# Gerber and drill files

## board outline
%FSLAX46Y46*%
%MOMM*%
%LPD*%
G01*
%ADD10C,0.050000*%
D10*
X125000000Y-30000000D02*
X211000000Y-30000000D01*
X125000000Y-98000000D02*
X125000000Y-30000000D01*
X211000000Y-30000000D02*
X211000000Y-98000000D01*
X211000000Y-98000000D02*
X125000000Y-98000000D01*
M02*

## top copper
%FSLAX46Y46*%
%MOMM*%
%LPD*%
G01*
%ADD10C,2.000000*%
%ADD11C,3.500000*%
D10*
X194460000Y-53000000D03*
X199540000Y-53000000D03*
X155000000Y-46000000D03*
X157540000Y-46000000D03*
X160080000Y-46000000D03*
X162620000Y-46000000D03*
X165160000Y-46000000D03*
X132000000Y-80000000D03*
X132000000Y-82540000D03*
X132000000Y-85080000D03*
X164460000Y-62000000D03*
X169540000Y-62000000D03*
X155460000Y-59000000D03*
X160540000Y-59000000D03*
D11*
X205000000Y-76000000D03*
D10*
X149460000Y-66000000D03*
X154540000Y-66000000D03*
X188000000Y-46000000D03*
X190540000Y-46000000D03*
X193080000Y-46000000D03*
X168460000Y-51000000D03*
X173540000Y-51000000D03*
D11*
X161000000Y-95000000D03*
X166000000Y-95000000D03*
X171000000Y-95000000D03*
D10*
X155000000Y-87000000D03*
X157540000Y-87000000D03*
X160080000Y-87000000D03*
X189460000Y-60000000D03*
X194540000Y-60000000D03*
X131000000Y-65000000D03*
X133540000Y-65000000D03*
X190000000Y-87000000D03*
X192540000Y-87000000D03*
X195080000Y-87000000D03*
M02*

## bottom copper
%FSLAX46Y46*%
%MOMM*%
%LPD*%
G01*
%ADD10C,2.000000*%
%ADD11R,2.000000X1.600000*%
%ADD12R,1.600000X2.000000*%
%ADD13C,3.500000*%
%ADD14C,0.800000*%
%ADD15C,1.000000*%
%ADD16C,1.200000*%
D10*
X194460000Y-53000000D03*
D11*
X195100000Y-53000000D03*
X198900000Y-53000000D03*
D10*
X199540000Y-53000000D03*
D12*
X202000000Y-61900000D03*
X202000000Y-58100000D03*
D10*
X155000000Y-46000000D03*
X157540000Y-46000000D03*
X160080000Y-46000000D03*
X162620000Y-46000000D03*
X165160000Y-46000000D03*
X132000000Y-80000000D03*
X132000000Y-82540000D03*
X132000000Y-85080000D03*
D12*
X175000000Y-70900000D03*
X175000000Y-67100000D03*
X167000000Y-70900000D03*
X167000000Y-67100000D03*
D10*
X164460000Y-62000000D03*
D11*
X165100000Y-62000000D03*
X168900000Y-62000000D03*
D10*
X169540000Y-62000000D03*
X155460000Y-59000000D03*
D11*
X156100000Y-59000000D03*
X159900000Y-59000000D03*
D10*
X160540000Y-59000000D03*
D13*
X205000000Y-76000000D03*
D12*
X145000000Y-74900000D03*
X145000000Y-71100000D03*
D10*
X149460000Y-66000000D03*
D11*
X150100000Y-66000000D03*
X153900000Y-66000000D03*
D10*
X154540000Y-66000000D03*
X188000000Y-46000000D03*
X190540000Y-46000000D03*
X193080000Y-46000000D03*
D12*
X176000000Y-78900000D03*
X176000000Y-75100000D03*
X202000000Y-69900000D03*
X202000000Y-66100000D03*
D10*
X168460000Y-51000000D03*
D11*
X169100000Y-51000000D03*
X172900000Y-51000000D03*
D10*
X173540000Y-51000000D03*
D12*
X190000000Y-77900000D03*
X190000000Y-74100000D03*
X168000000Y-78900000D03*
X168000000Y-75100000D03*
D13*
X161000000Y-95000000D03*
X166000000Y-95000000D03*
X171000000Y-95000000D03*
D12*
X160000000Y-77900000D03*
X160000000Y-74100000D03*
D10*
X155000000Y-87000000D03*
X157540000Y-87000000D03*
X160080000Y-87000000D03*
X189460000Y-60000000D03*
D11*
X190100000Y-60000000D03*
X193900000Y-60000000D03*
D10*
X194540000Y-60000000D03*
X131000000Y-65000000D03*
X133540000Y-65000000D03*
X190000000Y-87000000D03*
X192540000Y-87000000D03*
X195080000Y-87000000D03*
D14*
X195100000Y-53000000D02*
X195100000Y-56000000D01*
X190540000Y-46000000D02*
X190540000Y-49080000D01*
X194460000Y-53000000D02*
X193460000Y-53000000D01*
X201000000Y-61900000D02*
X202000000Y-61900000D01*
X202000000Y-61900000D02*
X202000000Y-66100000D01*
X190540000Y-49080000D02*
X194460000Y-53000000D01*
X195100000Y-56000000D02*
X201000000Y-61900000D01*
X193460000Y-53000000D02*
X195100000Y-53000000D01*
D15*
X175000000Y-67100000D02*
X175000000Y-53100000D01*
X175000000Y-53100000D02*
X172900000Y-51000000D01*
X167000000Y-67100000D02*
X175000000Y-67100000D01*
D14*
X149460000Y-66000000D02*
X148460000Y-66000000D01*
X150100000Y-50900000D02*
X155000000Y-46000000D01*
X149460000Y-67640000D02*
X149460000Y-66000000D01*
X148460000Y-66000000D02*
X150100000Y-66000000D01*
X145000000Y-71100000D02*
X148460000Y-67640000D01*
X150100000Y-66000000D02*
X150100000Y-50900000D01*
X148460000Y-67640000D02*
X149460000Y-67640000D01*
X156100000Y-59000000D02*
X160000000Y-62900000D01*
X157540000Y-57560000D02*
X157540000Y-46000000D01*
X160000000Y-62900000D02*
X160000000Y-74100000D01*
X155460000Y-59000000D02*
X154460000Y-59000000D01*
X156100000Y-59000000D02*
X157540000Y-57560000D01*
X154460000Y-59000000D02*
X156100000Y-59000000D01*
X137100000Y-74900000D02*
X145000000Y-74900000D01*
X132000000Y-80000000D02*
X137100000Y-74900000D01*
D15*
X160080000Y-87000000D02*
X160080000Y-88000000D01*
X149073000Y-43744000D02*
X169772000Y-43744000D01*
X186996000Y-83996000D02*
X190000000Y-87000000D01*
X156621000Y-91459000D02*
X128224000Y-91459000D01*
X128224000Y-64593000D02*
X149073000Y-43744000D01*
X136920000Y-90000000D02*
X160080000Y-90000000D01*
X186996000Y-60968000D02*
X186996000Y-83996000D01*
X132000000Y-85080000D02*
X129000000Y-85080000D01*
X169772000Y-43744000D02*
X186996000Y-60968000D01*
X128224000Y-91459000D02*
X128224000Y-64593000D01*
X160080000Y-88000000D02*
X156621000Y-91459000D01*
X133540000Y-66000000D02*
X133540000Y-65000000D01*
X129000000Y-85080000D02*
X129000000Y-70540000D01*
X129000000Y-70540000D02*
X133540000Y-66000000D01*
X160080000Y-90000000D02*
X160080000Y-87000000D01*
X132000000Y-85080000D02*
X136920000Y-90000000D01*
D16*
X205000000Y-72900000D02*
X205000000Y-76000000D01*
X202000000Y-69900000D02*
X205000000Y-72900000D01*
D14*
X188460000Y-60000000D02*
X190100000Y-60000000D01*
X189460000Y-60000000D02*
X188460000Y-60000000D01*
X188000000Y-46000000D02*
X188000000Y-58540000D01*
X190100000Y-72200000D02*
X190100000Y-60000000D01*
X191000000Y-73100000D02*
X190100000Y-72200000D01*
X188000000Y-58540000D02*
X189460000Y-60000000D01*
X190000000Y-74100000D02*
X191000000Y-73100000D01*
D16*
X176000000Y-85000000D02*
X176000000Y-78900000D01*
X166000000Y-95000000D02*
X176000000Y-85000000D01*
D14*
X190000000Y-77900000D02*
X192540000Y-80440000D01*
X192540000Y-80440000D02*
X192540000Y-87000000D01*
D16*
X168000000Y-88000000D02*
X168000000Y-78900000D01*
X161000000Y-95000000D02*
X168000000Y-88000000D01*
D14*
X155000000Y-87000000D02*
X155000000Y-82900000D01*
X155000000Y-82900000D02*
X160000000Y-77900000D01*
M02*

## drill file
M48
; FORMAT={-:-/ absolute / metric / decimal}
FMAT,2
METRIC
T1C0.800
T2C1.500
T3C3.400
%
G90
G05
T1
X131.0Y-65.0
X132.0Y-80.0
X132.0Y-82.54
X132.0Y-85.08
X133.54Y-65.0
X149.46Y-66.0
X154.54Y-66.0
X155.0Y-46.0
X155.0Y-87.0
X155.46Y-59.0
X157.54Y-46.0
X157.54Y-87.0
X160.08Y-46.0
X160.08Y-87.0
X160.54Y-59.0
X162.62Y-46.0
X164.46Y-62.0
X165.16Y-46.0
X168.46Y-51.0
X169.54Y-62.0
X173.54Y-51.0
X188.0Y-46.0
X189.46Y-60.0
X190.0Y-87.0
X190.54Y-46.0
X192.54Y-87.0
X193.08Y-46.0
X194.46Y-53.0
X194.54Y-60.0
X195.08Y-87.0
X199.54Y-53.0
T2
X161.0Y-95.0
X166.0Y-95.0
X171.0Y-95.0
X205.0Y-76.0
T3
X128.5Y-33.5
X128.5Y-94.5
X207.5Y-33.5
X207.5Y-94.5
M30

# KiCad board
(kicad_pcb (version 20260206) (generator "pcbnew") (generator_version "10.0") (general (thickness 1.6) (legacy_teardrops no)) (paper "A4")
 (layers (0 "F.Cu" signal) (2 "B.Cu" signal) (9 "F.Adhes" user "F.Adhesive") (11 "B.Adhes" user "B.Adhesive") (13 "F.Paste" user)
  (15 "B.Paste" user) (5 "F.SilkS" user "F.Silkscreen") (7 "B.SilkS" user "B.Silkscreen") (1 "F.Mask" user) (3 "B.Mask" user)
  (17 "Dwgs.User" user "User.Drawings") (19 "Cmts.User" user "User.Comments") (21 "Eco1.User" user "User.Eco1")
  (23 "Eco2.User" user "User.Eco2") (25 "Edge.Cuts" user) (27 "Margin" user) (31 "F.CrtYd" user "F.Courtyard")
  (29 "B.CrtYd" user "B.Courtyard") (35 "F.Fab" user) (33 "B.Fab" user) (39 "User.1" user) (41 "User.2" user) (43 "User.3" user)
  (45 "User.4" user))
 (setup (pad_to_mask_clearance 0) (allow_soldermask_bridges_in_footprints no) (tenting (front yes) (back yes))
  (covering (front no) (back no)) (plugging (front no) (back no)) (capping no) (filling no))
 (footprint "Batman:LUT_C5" (layer "F.Cu") (at 197 53)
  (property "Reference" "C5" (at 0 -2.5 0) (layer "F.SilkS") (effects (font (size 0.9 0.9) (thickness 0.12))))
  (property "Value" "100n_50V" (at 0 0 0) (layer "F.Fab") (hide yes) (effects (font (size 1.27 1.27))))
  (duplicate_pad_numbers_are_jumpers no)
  (pad "1" thru_hole circle (at -2.54 0) (size 2 2) (drill 0.8) (layers "*.Cu") (remove_unused_layers no) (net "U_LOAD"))
  (pad "1" smd rect (at -1.9 0) (size 2 1.6) (layers "B.Cu") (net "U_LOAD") (thermal_bridge_angle 45))
  (pad "2" smd rect (at 1.9 0) (size 2 1.6) (layers "B.Cu") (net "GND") (thermal_bridge_angle 45))
  (pad "2" thru_hole circle (at 2.54 0) (size 2 2) (drill 0.8) (layers "*.Cu") (remove_unused_layers no) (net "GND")))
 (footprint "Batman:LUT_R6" (layer "F.Cu") (at 202 60 90)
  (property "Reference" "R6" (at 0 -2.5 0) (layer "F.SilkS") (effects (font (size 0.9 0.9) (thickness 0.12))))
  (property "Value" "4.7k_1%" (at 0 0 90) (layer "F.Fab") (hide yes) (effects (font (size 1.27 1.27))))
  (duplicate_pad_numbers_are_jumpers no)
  (pad "1" smd rect (at -1.9 0 90) (size 2 1.6) (layers "B.Cu") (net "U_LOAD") (thermal_bridge_angle 45))
  (pad "2" smd rect (at 1.9 0 90) (size 2 1.6) (layers "B.Cu") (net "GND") (thermal_bridge_angle 45)))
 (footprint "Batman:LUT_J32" (layer "F.Cu") (at 155 46)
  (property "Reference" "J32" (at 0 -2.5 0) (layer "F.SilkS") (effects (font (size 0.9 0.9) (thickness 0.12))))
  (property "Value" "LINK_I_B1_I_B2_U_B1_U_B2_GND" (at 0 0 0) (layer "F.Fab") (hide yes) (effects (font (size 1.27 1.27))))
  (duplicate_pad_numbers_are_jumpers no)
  (pad "1" thru_hole circle (at 0 0) (size 2 2) (drill 0.8) (layers "*.Cu") (remove_unused_layers no) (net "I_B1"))
  (pad "2" thru_hole circle (at 2.54 0) (size 2 2) (drill 0.8) (layers "*.Cu") (remove_unused_layers no) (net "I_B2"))
  (pad "3" thru_hole circle (at 5.08 0) (size 2 2) (drill 0.8) (layers "*.Cu") (remove_unused_layers no) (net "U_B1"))
  (pad "4" thru_hole circle (at 7.62 0) (size 2 2) (drill 0.8) (layers "*.Cu") (remove_unused_layers no) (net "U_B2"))
  (pad "5" thru_hole circle (at 10.16 0) (size 2 2) (drill 0.8) (layers "*.Cu") (remove_unused_layers no) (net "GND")))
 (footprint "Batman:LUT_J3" (layer "F.Cu") (at 132 80 -90)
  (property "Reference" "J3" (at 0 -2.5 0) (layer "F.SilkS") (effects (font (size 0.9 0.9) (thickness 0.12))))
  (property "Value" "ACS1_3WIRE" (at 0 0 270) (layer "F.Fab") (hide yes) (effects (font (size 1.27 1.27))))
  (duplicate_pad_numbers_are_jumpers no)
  (pad "1" thru_hole circle (at 0 0 270) (size 2 2) (drill 0.8) (layers "*.Cu") (remove_unused_layers no) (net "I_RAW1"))
  (pad "2" thru_hole circle (at 2.54 0 270) (size 2 2) (drill 0.8) (layers "*.Cu") (remove_unused_layers no) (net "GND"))
  (pad "3" thru_hole circle (at 5.08 0 270) (size 2 2) (drill 0.8) (layers "*.Cu") (remove_unused_layers no) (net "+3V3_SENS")))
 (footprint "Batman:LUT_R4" (layer "F.Cu") (at 175 69 90)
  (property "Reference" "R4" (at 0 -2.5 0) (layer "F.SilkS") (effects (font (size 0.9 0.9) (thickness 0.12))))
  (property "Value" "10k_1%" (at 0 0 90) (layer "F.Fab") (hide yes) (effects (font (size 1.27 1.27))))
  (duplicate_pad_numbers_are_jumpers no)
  (pad "1" smd rect (at -1.9 0 90) (size 2 1.6) (layers "B.Cu") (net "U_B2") (thermal_bridge_angle 45))
  (pad "2" smd rect (at 1.9 0 90) (size 2 1.6) (layers "B.Cu") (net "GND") (thermal_bridge_angle 45)))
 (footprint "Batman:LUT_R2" (layer "F.Cu") (at 167 69 90)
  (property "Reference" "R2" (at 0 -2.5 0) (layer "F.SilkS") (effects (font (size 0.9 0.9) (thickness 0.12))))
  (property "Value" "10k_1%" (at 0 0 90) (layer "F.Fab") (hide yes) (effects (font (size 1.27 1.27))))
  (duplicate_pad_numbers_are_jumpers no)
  (pad "1" smd rect (at -1.9 0 90) (size 2 1.6) (layers "B.Cu") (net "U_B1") (thermal_bridge_angle 45))
  (pad "2" smd rect (at 1.9 0 90) (size 2 1.6) (layers "B.Cu") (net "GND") (thermal_bridge_angle 45)))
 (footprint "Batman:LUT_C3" (layer "F.Cu") (at 167 62)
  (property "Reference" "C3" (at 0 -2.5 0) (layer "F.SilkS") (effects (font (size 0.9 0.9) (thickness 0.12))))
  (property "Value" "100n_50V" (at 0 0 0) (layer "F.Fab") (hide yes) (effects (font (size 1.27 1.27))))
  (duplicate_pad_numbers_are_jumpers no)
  (pad "1" thru_hole circle (at -2.54 0) (size 2 2) (drill 0.8) (layers "*.Cu") (remove_unused_layers no) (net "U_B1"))
  (pad "1" smd rect (at -1.9 0) (size 2 1.6) (layers "B.Cu") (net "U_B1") (thermal_bridge_angle 45))
  (pad "2" smd rect (at 1.9 0) (size 2 1.6) (layers "B.Cu") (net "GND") (thermal_bridge_angle 45))
  (pad "2" thru_hole circle (at 2.54 0) (size 2 2) (drill 0.8) (layers "*.Cu") (remove_unused_layers no) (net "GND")))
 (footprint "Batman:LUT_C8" (layer "F.Cu") (at 158 59)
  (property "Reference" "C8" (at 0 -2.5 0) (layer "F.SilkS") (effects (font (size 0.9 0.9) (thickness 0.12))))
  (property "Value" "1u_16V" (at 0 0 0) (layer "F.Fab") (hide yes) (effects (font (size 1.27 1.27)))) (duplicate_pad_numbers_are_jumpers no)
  (pad "1" thru_hole circle (at -2.54 0) (size 2 2) (drill 0.8) (layers "*.Cu") (remove_unused_layers no) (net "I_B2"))
  (pad "1" smd rect (at -1.9 0) (size 2 1.6) (layers "B.Cu") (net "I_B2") (thermal_bridge_angle 45))
  (pad "2" smd rect (at 1.9 0) (size 2 1.6) (layers "B.Cu") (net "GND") (thermal_bridge_angle 45))
  (pad "2" thru_hole circle (at 2.54 0) (size 2 2) (drill 0.8) (layers "*.Cu") (remove_unused_layers no) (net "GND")))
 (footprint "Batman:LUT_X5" (layer "F.Cu") (at 205 76)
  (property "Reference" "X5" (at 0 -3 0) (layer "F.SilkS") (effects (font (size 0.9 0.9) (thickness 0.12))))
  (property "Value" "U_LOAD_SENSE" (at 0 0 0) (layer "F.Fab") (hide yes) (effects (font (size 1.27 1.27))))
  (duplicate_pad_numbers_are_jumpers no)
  (pad "1" thru_hole circle (at 0 0) (size 3.5 3.5) (drill 1.5) (layers "*.Cu") (remove_unused_layers no) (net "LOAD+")))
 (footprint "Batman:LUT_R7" (layer "F.Cu") (at 145 73 90)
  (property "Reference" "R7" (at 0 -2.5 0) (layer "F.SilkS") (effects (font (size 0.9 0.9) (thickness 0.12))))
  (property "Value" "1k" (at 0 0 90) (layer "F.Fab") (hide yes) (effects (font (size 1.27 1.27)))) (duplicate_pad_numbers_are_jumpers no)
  (pad "1" smd rect (at -1.9 0 90) (size 2 1.6) (layers "B.Cu") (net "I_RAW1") (thermal_bridge_angle 45))
  (pad "2" smd rect (at 1.9 0 90) (size 2 1.6) (layers "B.Cu") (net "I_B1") (thermal_bridge_angle 45)))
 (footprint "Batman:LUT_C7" (layer "F.Cu") (at 152 66)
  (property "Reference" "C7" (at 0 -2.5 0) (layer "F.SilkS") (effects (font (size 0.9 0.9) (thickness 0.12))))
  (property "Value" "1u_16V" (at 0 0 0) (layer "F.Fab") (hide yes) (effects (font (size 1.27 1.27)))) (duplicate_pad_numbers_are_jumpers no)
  (pad "1" thru_hole circle (at -2.54 0) (size 2 2) (drill 0.8) (layers "*.Cu") (remove_unused_layers no) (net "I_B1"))
  (pad "1" smd rect (at -1.9 0) (size 2 1.6) (layers "B.Cu") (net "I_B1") (thermal_bridge_angle 45))
  (pad "2" smd rect (at 1.9 0) (size 2 1.6) (layers "B.Cu") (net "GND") (thermal_bridge_angle 45))
  (pad "2" thru_hole circle (at 2.54 0) (size 2 2) (drill 0.8) (layers "*.Cu") (remove_unused_layers no) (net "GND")))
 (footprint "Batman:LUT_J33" (layer "F.Cu") (at 188 46)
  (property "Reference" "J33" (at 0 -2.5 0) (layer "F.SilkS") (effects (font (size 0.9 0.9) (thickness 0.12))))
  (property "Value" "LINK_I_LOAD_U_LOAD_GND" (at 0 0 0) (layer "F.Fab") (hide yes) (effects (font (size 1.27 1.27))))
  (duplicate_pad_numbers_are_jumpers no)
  (pad "1" thru_hole circle (at 0 0) (size 2 2) (drill 0.8) (layers "*.Cu") (remove_unused_layers no) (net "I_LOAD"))
  (pad "2" thru_hole circle (at 2.54 0) (size 2 2) (drill 0.8) (layers "*.Cu") (remove_unused_layers no) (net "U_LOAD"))
  (pad "3" thru_hole circle (at 5.08 0) (size 2 2) (drill 0.8) (layers "*.Cu") (remove_unused_layers no) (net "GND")))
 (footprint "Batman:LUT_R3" (layer "F.Cu") (at 176 77 90)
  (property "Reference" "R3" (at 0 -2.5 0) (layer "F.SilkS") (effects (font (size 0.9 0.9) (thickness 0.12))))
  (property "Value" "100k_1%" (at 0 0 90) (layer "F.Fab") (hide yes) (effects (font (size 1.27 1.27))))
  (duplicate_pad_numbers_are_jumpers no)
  (pad "1" smd rect (at -1.9 0 90) (size 2 1.6) (layers "B.Cu") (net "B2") (thermal_bridge_angle 45))
  (pad "2" smd rect (at 1.9 0 90) (size 2 1.6) (layers "B.Cu") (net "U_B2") (thermal_bridge_angle 45)))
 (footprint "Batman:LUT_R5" (layer "F.Cu") (at 202 68 90)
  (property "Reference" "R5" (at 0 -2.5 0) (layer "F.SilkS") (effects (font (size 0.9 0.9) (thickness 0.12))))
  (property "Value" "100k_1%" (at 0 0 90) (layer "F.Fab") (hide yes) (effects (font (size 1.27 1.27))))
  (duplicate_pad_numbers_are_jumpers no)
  (pad "1" smd rect (at -1.9 0 90) (size 2 1.6) (layers "B.Cu") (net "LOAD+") (thermal_bridge_angle 45))
  (pad "2" smd rect (at 1.9 0 90) (size 2 1.6) (layers "B.Cu") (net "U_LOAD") (thermal_bridge_angle 45)))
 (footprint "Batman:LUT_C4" (layer "F.Cu") (at 171 51)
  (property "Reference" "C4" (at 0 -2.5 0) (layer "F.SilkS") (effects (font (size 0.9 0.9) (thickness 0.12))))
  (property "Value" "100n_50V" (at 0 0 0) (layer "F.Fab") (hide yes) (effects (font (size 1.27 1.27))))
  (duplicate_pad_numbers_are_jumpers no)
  (pad "1" thru_hole circle (at -2.54 0) (size 2 2) (drill 0.8) (layers "*.Cu") (remove_unused_layers no) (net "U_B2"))
  (pad "1" smd rect (at -1.9 0) (size 2 1.6) (layers "B.Cu") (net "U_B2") (thermal_bridge_angle 45))
  (pad "2" smd rect (at 1.9 0) (size 2 1.6) (layers "B.Cu") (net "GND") (thermal_bridge_angle 45))
  (pad "2" thru_hole circle (at 2.54 0) (size 2 2) (drill 0.8) (layers "*.Cu") (remove_unused_layers no) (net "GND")))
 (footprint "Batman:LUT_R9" (layer "F.Cu") (at 190 76 90)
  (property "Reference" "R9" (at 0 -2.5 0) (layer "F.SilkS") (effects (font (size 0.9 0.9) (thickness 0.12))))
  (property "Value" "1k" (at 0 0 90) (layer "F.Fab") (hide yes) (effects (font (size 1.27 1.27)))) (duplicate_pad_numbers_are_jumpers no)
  (pad "1" smd rect (at -1.9 0 90) (size 2 1.6) (layers "B.Cu") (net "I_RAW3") (thermal_bridge_angle 45))
  (pad "2" smd rect (at 1.9 0 90) (size 2 1.6) (layers "B.Cu") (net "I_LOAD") (thermal_bridge_angle 45)))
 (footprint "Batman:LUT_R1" (layer "F.Cu") (at 168 77 90)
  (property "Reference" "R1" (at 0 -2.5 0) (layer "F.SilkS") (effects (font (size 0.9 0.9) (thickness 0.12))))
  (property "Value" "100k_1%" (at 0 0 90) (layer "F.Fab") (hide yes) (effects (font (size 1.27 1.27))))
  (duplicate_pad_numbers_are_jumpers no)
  (pad "1" smd rect (at -1.9 0 90) (size 2 1.6) (layers "B.Cu") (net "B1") (thermal_bridge_angle 45))
  (pad "2" smd rect (at 1.9 0 90) (size 2 1.6) (layers "B.Cu") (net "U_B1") (thermal_bridge_angle 45)))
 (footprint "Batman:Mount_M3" (layer "F.Cu") (at 207.5 33.5)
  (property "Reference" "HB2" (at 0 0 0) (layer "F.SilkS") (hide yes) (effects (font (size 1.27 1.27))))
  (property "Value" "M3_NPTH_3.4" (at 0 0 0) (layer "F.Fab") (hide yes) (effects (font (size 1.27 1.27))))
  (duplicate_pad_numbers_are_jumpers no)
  (pad "" np_thru_hole circle (at 0 0) (size 3.4 3.4) (drill 3.4) (layers "*.Cu")))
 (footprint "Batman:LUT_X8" (layer "F.Cu") (at 161 95)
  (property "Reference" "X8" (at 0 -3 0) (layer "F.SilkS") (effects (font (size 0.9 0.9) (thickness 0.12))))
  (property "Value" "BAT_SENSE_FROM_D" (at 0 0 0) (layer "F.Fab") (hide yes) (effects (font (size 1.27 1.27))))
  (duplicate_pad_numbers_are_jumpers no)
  (pad "1" thru_hole circle (at 0 0) (size 3.5 3.5) (drill 1.5) (layers "*.Cu") (remove_unused_layers no) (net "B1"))
  (pad "2" thru_hole circle (at 5 0) (size 3.5 3.5) (drill 1.5) (layers "*.Cu") (remove_unused_layers no) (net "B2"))
  (pad "3" thru_hole circle (at 10 0) (size 3.5 3.5) (drill 1.5) (layers "*.Cu") (remove_unused_layers no) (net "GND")))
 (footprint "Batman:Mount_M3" (layer "F.Cu") (at 207.5 94.5)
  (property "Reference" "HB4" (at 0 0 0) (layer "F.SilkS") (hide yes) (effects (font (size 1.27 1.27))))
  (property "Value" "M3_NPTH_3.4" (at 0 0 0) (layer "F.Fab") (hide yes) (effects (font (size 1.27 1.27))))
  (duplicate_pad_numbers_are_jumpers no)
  (pad "" np_thru_hole circle (at 0 0) (size 3.4 3.4) (drill 3.4) (layers "*.Cu")))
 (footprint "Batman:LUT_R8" (layer "F.Cu") (at 160 76 90)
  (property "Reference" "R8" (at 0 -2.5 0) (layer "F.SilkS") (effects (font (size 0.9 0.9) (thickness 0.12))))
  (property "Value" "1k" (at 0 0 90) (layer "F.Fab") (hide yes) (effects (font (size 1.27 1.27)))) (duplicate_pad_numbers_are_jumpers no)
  (pad "1" smd rect (at -1.9 0 90) (size 2 1.6) (layers "B.Cu") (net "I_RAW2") (thermal_bridge_angle 45))
  (pad "2" smd rect (at 1.9 0 90) (size 2 1.6) (layers "B.Cu") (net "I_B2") (thermal_bridge_angle 45)))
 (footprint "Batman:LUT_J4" (layer "F.Cu") (at 155 87)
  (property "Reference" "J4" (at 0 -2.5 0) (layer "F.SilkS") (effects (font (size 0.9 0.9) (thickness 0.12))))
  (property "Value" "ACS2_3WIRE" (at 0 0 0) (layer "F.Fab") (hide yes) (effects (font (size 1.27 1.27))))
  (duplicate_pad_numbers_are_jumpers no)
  (pad "1" thru_hole circle (at 0 0) (size 2 2) (drill 0.8) (layers "*.Cu") (remove_unused_layers no) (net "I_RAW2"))
  (pad "2" thru_hole circle (at 2.54 0) (size 2 2) (drill 0.8) (layers "*.Cu") (remove_unused_layers no) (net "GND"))
  (pad "3" thru_hole circle (at 5.08 0) (size 2 2) (drill 0.8) (layers "*.Cu") (remove_unused_layers no) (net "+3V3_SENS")))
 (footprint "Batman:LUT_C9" (layer "F.Cu") (at 192 60)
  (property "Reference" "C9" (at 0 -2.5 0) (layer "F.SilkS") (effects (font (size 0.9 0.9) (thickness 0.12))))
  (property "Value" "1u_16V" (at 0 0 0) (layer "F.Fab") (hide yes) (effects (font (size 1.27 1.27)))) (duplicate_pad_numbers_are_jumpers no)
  (pad "1" thru_hole circle (at -2.54 0) (size 2 2) (drill 0.8) (layers "*.Cu") (remove_unused_layers no) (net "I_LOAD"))
  (pad "1" smd rect (at -1.9 0) (size 2 1.6) (layers "B.Cu") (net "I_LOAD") (thermal_bridge_angle 45))
  (pad "2" smd rect (at 1.9 0) (size 2 1.6) (layers "B.Cu") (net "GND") (thermal_bridge_angle 45))
  (pad "2" thru_hole circle (at 2.54 0) (size 2 2) (drill 0.8) (layers "*.Cu") (remove_unused_layers no) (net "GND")))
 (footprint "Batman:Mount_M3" (layer "F.Cu") (at 128.5 33.5)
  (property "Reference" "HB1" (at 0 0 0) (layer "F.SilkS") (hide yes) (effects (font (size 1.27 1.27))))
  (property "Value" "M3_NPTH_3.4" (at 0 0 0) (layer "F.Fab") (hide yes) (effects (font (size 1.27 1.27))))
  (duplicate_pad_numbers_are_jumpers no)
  (pad "" np_thru_hole circle (at 0 0) (size 3.4 3.4) (drill 3.4) (layers "*.Cu")))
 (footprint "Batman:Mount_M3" (layer "F.Cu") (at 128.5 94.5)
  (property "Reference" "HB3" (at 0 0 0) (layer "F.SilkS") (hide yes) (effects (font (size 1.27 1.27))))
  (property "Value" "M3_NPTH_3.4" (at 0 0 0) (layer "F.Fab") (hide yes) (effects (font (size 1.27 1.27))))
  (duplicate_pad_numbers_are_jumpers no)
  (pad "" np_thru_hole circle (at 0 0) (size 3.4 3.4) (drill 3.4) (layers "*.Cu")))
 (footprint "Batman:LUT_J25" (layer "F.Cu") (at 131 65)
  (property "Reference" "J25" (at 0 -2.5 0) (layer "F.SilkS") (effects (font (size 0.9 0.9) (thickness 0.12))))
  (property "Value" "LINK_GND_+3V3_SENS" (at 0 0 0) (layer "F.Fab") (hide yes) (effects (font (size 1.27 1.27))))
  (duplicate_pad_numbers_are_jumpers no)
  (pad "1" thru_hole circle (at 0 0) (size 2 2) (drill 0.8) (layers "*.Cu") (remove_unused_layers no) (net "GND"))
  (pad "2" thru_hole circle (at 2.54 0) (size 2 2) (drill 0.8) (layers "*.Cu") (remove_unused_layers no) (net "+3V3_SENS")))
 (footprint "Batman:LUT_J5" (layer "F.Cu") (at 190 87)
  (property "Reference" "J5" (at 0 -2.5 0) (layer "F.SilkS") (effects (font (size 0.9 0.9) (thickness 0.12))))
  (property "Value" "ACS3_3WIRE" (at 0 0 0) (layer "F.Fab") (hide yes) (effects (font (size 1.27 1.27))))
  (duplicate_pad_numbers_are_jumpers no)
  (pad "1" thru_hole circle (at 0 0) (size 2 2) (drill 0.8) (layers "*.Cu") (remove_unused_layers no) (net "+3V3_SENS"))
  (pad "2" thru_hole circle (at 2.54 0) (size 2 2) (drill 0.8) (layers "*.Cu") (remove_unused_layers no) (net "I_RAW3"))
  (pad "3" thru_hole circle (at 5.08 0) (size 2 2) (drill 0.8) (layers "*.Cu") (remove_unused_layers no) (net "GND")))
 (gr_line (start 125 30) (end 211 30) (stroke (width 0.05) (type default)) (layer "Edge.Cuts"))
 (gr_line (start 125 98) (end 125 30) (stroke (width 0.05) (type default)) (layer "Edge.Cuts"))
 (gr_line (start 211 30) (end 211 98) (stroke (width 0.05) (type default)) (layer "Edge.Cuts"))
 (gr_line (start 211 98) (end 125 98) (stroke (width 0.05) (type default)) (layer "Edge.Cuts"))
 (segment (start 195.1 53) (end 195.1 56) (width 0.8) (layer "B.Cu") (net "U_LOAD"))
 (segment (start 190.54 46) (end 190.54 49.08) (width 0.8) (layer "B.Cu") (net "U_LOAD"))
 (segment (start 194.46 53) (end 193.46 53) (width 0.8) (layer "B.Cu") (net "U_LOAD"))
 (segment (start 201 61.9) (end 202 61.9) (width 0.8) (layer "B.Cu") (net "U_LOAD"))
 (segment (start 202 61.9) (end 202 66.1) (width 0.8) (layer "B.Cu") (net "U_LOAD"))
 (segment (start 190.54 49.08) (end 194.46 53) (width 0.8) (layer "B.Cu") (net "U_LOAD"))
 (segment (start 195.1 56) (end 201 61.9) (width 0.8) (layer "B.Cu") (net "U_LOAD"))
 (segment (start 193.46 53) (end 195.1 53) (width 0.8) (layer "B.Cu") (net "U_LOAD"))
 (segment (start 175 67.1) (end 175 53.1) (width 1) (layer "B.Cu") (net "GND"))
 (segment (start 175 53.1) (end 172.9 51) (width 1) (layer "B.Cu") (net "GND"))
 (segment (start 167 67.1) (end 175 67.1) (width 1) (layer "B.Cu") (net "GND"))
 (segment (start 149.46 66) (end 148.46 66) (width 0.8) (layer "B.Cu") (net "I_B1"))
 (segment (start 150.1 50.9) (end 155 46) (width 0.8) (layer "B.Cu") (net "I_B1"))
 (segment (start 149.46 67.64) (end 149.46 66) (width 0.8) (layer "B.Cu") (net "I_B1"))
 (segment (start 148.46 66) (end 150.1 66) (width 0.8) (layer "B.Cu") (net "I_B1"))
 (segment (start 145 71.1) (end 148.46 67.64) (width 0.8) (layer "B.Cu") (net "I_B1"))
 (segment (start 150.1 66) (end 150.1 50.9) (width 0.8) (layer "B.Cu") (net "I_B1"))
 (segment (start 148.46 67.64) (end 149.46 67.64) (width 0.8) (layer "B.Cu") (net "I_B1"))
 (segment (start 156.1 59) (end 160 62.9) (width 0.8) (layer "B.Cu") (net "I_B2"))
 (segment (start 157.54 57.56) (end 157.54 46) (width 0.8) (layer "B.Cu") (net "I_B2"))
 (segment (start 160 62.9) (end 160 74.1) (width 0.8) (layer "B.Cu") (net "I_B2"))
 (segment (start 155.46 59) (end 154.46 59) (width 0.8) (layer "B.Cu") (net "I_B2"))
 (segment (start 156.1 59) (end 157.54 57.56) (width 0.8) (layer "B.Cu") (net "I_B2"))
 (segment (start 154.46 59) (end 156.1 59) (width 0.8) (layer "B.Cu") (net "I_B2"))
 (segment (start 137.1 74.9) (end 145 74.9) (width 0.8) (layer "B.Cu") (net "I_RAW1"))
 (segment (start 132 80) (end 137.1 74.9) (width 0.8) (layer "B.Cu") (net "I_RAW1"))
 (segment (start 160.08 87) (end 160.08 88) (width 1) (layer "B.Cu") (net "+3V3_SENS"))
 (segment (start 149.073 43.744) (end 169.772 43.744) (width 1) (layer "B.Cu") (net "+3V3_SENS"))
 (segment (start 186.996 83.996) (end 190 87) (width 1) (layer "B.Cu") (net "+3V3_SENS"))
 (segment (start 156.621 91.459) (end 128.224 91.459) (width 1) (layer "B.Cu") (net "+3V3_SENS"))
 (segment (start 128.224 64.593) (end 149.073 43.744) (width 1) (layer "B.Cu") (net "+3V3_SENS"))
 (segment (start 136.92 90) (end 160.08 90) (width 1) (layer "B.Cu") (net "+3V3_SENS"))
 (segment (start 186.996 60.968) (end 186.996 83.996) (width 1) (layer "B.Cu") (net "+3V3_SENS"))
 (segment (start 132 85.08) (end 129 85.08) (width 1) (layer "B.Cu") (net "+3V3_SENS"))
 (segment (start 169.772 43.744) (end 186.996 60.968) (width 1) (layer "B.Cu") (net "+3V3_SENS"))
 (segment (start 128.224 91.459) (end 128.224 64.593) (width 1) (layer "B.Cu") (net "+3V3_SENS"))
 (segment (start 160.08 88) (end 156.621 91.459) (width 1) (layer "B.Cu") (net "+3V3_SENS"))
 (segment (start 133.54 66) (end 133.54 65) (width 1) (layer "B.Cu") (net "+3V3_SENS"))
 (segment (start 129 85.08) (end 129 70.54) (width 1) (layer "B.Cu") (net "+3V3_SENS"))
 (segment (start 129 70.54) (end 133.54 66) (width 1) (layer "B.Cu") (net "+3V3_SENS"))
 (segment (start 160.08 90) (end 160.08 87) (width 1) (layer "B.Cu") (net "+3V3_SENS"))
 (segment (start 132 85.08) (end 136.92 90) (width 1) (layer "B.Cu") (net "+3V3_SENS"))
 (segment (start 205 72.9) (end 205 76) (width 1.2) (layer "B.Cu") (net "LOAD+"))
 (segment (start 202 69.9) (end 205 72.9) (width 1.2) (layer "B.Cu") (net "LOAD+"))
 (segment (start 188.46 60) (end 190.1 60) (width 0.8) (layer "B.Cu") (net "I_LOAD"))
 (segment (start 189.46 60) (end 188.46 60) (width 0.8) (layer "B.Cu") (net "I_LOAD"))
 (segment (start 188 46) (end 188 58.54) (width 0.8) (layer "B.Cu") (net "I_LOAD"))
 (segment (start 190.1 72.2) (end 190.1 60) (width 0.8) (layer "B.Cu") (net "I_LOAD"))
 (segment (start 191 73.1) (end 190.1 72.2) (width 0.8) (layer "B.Cu") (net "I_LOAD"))
 (segment (start 188 58.54) (end 189.46 60) (width 0.8) (layer "B.Cu") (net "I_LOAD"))
 (segment (start 190 74.1) (end 191 73.1) (width 0.8) (layer "B.Cu") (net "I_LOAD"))
 (segment (start 176 85) (end 176 78.9) (width 1.2) (layer "B.Cu") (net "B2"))
 (segment (start 166 95) (end 176 85) (width 1.2) (layer "B.Cu") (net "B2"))
 (segment (start 190 77.9) (end 192.54 80.44) (width 0.8) (layer "B.Cu") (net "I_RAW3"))
 (segment (start 192.54 80.44) (end 192.54 87) (width 0.8) (layer "B.Cu") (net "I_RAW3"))
 (segment (start 168 88) (end 168 78.9) (width 1.2) (layer "B.Cu") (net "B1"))
 (segment (start 161 95) (end 168 88) (width 1.2) (layer "B.Cu") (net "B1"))
 (segment (start 155 87) (end 155 82.9) (width 0.8) (layer "B.Cu") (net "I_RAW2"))
 (segment (start 155 82.9) (end 160 77.9) (width 0.8) (layer "B.Cu") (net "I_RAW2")))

